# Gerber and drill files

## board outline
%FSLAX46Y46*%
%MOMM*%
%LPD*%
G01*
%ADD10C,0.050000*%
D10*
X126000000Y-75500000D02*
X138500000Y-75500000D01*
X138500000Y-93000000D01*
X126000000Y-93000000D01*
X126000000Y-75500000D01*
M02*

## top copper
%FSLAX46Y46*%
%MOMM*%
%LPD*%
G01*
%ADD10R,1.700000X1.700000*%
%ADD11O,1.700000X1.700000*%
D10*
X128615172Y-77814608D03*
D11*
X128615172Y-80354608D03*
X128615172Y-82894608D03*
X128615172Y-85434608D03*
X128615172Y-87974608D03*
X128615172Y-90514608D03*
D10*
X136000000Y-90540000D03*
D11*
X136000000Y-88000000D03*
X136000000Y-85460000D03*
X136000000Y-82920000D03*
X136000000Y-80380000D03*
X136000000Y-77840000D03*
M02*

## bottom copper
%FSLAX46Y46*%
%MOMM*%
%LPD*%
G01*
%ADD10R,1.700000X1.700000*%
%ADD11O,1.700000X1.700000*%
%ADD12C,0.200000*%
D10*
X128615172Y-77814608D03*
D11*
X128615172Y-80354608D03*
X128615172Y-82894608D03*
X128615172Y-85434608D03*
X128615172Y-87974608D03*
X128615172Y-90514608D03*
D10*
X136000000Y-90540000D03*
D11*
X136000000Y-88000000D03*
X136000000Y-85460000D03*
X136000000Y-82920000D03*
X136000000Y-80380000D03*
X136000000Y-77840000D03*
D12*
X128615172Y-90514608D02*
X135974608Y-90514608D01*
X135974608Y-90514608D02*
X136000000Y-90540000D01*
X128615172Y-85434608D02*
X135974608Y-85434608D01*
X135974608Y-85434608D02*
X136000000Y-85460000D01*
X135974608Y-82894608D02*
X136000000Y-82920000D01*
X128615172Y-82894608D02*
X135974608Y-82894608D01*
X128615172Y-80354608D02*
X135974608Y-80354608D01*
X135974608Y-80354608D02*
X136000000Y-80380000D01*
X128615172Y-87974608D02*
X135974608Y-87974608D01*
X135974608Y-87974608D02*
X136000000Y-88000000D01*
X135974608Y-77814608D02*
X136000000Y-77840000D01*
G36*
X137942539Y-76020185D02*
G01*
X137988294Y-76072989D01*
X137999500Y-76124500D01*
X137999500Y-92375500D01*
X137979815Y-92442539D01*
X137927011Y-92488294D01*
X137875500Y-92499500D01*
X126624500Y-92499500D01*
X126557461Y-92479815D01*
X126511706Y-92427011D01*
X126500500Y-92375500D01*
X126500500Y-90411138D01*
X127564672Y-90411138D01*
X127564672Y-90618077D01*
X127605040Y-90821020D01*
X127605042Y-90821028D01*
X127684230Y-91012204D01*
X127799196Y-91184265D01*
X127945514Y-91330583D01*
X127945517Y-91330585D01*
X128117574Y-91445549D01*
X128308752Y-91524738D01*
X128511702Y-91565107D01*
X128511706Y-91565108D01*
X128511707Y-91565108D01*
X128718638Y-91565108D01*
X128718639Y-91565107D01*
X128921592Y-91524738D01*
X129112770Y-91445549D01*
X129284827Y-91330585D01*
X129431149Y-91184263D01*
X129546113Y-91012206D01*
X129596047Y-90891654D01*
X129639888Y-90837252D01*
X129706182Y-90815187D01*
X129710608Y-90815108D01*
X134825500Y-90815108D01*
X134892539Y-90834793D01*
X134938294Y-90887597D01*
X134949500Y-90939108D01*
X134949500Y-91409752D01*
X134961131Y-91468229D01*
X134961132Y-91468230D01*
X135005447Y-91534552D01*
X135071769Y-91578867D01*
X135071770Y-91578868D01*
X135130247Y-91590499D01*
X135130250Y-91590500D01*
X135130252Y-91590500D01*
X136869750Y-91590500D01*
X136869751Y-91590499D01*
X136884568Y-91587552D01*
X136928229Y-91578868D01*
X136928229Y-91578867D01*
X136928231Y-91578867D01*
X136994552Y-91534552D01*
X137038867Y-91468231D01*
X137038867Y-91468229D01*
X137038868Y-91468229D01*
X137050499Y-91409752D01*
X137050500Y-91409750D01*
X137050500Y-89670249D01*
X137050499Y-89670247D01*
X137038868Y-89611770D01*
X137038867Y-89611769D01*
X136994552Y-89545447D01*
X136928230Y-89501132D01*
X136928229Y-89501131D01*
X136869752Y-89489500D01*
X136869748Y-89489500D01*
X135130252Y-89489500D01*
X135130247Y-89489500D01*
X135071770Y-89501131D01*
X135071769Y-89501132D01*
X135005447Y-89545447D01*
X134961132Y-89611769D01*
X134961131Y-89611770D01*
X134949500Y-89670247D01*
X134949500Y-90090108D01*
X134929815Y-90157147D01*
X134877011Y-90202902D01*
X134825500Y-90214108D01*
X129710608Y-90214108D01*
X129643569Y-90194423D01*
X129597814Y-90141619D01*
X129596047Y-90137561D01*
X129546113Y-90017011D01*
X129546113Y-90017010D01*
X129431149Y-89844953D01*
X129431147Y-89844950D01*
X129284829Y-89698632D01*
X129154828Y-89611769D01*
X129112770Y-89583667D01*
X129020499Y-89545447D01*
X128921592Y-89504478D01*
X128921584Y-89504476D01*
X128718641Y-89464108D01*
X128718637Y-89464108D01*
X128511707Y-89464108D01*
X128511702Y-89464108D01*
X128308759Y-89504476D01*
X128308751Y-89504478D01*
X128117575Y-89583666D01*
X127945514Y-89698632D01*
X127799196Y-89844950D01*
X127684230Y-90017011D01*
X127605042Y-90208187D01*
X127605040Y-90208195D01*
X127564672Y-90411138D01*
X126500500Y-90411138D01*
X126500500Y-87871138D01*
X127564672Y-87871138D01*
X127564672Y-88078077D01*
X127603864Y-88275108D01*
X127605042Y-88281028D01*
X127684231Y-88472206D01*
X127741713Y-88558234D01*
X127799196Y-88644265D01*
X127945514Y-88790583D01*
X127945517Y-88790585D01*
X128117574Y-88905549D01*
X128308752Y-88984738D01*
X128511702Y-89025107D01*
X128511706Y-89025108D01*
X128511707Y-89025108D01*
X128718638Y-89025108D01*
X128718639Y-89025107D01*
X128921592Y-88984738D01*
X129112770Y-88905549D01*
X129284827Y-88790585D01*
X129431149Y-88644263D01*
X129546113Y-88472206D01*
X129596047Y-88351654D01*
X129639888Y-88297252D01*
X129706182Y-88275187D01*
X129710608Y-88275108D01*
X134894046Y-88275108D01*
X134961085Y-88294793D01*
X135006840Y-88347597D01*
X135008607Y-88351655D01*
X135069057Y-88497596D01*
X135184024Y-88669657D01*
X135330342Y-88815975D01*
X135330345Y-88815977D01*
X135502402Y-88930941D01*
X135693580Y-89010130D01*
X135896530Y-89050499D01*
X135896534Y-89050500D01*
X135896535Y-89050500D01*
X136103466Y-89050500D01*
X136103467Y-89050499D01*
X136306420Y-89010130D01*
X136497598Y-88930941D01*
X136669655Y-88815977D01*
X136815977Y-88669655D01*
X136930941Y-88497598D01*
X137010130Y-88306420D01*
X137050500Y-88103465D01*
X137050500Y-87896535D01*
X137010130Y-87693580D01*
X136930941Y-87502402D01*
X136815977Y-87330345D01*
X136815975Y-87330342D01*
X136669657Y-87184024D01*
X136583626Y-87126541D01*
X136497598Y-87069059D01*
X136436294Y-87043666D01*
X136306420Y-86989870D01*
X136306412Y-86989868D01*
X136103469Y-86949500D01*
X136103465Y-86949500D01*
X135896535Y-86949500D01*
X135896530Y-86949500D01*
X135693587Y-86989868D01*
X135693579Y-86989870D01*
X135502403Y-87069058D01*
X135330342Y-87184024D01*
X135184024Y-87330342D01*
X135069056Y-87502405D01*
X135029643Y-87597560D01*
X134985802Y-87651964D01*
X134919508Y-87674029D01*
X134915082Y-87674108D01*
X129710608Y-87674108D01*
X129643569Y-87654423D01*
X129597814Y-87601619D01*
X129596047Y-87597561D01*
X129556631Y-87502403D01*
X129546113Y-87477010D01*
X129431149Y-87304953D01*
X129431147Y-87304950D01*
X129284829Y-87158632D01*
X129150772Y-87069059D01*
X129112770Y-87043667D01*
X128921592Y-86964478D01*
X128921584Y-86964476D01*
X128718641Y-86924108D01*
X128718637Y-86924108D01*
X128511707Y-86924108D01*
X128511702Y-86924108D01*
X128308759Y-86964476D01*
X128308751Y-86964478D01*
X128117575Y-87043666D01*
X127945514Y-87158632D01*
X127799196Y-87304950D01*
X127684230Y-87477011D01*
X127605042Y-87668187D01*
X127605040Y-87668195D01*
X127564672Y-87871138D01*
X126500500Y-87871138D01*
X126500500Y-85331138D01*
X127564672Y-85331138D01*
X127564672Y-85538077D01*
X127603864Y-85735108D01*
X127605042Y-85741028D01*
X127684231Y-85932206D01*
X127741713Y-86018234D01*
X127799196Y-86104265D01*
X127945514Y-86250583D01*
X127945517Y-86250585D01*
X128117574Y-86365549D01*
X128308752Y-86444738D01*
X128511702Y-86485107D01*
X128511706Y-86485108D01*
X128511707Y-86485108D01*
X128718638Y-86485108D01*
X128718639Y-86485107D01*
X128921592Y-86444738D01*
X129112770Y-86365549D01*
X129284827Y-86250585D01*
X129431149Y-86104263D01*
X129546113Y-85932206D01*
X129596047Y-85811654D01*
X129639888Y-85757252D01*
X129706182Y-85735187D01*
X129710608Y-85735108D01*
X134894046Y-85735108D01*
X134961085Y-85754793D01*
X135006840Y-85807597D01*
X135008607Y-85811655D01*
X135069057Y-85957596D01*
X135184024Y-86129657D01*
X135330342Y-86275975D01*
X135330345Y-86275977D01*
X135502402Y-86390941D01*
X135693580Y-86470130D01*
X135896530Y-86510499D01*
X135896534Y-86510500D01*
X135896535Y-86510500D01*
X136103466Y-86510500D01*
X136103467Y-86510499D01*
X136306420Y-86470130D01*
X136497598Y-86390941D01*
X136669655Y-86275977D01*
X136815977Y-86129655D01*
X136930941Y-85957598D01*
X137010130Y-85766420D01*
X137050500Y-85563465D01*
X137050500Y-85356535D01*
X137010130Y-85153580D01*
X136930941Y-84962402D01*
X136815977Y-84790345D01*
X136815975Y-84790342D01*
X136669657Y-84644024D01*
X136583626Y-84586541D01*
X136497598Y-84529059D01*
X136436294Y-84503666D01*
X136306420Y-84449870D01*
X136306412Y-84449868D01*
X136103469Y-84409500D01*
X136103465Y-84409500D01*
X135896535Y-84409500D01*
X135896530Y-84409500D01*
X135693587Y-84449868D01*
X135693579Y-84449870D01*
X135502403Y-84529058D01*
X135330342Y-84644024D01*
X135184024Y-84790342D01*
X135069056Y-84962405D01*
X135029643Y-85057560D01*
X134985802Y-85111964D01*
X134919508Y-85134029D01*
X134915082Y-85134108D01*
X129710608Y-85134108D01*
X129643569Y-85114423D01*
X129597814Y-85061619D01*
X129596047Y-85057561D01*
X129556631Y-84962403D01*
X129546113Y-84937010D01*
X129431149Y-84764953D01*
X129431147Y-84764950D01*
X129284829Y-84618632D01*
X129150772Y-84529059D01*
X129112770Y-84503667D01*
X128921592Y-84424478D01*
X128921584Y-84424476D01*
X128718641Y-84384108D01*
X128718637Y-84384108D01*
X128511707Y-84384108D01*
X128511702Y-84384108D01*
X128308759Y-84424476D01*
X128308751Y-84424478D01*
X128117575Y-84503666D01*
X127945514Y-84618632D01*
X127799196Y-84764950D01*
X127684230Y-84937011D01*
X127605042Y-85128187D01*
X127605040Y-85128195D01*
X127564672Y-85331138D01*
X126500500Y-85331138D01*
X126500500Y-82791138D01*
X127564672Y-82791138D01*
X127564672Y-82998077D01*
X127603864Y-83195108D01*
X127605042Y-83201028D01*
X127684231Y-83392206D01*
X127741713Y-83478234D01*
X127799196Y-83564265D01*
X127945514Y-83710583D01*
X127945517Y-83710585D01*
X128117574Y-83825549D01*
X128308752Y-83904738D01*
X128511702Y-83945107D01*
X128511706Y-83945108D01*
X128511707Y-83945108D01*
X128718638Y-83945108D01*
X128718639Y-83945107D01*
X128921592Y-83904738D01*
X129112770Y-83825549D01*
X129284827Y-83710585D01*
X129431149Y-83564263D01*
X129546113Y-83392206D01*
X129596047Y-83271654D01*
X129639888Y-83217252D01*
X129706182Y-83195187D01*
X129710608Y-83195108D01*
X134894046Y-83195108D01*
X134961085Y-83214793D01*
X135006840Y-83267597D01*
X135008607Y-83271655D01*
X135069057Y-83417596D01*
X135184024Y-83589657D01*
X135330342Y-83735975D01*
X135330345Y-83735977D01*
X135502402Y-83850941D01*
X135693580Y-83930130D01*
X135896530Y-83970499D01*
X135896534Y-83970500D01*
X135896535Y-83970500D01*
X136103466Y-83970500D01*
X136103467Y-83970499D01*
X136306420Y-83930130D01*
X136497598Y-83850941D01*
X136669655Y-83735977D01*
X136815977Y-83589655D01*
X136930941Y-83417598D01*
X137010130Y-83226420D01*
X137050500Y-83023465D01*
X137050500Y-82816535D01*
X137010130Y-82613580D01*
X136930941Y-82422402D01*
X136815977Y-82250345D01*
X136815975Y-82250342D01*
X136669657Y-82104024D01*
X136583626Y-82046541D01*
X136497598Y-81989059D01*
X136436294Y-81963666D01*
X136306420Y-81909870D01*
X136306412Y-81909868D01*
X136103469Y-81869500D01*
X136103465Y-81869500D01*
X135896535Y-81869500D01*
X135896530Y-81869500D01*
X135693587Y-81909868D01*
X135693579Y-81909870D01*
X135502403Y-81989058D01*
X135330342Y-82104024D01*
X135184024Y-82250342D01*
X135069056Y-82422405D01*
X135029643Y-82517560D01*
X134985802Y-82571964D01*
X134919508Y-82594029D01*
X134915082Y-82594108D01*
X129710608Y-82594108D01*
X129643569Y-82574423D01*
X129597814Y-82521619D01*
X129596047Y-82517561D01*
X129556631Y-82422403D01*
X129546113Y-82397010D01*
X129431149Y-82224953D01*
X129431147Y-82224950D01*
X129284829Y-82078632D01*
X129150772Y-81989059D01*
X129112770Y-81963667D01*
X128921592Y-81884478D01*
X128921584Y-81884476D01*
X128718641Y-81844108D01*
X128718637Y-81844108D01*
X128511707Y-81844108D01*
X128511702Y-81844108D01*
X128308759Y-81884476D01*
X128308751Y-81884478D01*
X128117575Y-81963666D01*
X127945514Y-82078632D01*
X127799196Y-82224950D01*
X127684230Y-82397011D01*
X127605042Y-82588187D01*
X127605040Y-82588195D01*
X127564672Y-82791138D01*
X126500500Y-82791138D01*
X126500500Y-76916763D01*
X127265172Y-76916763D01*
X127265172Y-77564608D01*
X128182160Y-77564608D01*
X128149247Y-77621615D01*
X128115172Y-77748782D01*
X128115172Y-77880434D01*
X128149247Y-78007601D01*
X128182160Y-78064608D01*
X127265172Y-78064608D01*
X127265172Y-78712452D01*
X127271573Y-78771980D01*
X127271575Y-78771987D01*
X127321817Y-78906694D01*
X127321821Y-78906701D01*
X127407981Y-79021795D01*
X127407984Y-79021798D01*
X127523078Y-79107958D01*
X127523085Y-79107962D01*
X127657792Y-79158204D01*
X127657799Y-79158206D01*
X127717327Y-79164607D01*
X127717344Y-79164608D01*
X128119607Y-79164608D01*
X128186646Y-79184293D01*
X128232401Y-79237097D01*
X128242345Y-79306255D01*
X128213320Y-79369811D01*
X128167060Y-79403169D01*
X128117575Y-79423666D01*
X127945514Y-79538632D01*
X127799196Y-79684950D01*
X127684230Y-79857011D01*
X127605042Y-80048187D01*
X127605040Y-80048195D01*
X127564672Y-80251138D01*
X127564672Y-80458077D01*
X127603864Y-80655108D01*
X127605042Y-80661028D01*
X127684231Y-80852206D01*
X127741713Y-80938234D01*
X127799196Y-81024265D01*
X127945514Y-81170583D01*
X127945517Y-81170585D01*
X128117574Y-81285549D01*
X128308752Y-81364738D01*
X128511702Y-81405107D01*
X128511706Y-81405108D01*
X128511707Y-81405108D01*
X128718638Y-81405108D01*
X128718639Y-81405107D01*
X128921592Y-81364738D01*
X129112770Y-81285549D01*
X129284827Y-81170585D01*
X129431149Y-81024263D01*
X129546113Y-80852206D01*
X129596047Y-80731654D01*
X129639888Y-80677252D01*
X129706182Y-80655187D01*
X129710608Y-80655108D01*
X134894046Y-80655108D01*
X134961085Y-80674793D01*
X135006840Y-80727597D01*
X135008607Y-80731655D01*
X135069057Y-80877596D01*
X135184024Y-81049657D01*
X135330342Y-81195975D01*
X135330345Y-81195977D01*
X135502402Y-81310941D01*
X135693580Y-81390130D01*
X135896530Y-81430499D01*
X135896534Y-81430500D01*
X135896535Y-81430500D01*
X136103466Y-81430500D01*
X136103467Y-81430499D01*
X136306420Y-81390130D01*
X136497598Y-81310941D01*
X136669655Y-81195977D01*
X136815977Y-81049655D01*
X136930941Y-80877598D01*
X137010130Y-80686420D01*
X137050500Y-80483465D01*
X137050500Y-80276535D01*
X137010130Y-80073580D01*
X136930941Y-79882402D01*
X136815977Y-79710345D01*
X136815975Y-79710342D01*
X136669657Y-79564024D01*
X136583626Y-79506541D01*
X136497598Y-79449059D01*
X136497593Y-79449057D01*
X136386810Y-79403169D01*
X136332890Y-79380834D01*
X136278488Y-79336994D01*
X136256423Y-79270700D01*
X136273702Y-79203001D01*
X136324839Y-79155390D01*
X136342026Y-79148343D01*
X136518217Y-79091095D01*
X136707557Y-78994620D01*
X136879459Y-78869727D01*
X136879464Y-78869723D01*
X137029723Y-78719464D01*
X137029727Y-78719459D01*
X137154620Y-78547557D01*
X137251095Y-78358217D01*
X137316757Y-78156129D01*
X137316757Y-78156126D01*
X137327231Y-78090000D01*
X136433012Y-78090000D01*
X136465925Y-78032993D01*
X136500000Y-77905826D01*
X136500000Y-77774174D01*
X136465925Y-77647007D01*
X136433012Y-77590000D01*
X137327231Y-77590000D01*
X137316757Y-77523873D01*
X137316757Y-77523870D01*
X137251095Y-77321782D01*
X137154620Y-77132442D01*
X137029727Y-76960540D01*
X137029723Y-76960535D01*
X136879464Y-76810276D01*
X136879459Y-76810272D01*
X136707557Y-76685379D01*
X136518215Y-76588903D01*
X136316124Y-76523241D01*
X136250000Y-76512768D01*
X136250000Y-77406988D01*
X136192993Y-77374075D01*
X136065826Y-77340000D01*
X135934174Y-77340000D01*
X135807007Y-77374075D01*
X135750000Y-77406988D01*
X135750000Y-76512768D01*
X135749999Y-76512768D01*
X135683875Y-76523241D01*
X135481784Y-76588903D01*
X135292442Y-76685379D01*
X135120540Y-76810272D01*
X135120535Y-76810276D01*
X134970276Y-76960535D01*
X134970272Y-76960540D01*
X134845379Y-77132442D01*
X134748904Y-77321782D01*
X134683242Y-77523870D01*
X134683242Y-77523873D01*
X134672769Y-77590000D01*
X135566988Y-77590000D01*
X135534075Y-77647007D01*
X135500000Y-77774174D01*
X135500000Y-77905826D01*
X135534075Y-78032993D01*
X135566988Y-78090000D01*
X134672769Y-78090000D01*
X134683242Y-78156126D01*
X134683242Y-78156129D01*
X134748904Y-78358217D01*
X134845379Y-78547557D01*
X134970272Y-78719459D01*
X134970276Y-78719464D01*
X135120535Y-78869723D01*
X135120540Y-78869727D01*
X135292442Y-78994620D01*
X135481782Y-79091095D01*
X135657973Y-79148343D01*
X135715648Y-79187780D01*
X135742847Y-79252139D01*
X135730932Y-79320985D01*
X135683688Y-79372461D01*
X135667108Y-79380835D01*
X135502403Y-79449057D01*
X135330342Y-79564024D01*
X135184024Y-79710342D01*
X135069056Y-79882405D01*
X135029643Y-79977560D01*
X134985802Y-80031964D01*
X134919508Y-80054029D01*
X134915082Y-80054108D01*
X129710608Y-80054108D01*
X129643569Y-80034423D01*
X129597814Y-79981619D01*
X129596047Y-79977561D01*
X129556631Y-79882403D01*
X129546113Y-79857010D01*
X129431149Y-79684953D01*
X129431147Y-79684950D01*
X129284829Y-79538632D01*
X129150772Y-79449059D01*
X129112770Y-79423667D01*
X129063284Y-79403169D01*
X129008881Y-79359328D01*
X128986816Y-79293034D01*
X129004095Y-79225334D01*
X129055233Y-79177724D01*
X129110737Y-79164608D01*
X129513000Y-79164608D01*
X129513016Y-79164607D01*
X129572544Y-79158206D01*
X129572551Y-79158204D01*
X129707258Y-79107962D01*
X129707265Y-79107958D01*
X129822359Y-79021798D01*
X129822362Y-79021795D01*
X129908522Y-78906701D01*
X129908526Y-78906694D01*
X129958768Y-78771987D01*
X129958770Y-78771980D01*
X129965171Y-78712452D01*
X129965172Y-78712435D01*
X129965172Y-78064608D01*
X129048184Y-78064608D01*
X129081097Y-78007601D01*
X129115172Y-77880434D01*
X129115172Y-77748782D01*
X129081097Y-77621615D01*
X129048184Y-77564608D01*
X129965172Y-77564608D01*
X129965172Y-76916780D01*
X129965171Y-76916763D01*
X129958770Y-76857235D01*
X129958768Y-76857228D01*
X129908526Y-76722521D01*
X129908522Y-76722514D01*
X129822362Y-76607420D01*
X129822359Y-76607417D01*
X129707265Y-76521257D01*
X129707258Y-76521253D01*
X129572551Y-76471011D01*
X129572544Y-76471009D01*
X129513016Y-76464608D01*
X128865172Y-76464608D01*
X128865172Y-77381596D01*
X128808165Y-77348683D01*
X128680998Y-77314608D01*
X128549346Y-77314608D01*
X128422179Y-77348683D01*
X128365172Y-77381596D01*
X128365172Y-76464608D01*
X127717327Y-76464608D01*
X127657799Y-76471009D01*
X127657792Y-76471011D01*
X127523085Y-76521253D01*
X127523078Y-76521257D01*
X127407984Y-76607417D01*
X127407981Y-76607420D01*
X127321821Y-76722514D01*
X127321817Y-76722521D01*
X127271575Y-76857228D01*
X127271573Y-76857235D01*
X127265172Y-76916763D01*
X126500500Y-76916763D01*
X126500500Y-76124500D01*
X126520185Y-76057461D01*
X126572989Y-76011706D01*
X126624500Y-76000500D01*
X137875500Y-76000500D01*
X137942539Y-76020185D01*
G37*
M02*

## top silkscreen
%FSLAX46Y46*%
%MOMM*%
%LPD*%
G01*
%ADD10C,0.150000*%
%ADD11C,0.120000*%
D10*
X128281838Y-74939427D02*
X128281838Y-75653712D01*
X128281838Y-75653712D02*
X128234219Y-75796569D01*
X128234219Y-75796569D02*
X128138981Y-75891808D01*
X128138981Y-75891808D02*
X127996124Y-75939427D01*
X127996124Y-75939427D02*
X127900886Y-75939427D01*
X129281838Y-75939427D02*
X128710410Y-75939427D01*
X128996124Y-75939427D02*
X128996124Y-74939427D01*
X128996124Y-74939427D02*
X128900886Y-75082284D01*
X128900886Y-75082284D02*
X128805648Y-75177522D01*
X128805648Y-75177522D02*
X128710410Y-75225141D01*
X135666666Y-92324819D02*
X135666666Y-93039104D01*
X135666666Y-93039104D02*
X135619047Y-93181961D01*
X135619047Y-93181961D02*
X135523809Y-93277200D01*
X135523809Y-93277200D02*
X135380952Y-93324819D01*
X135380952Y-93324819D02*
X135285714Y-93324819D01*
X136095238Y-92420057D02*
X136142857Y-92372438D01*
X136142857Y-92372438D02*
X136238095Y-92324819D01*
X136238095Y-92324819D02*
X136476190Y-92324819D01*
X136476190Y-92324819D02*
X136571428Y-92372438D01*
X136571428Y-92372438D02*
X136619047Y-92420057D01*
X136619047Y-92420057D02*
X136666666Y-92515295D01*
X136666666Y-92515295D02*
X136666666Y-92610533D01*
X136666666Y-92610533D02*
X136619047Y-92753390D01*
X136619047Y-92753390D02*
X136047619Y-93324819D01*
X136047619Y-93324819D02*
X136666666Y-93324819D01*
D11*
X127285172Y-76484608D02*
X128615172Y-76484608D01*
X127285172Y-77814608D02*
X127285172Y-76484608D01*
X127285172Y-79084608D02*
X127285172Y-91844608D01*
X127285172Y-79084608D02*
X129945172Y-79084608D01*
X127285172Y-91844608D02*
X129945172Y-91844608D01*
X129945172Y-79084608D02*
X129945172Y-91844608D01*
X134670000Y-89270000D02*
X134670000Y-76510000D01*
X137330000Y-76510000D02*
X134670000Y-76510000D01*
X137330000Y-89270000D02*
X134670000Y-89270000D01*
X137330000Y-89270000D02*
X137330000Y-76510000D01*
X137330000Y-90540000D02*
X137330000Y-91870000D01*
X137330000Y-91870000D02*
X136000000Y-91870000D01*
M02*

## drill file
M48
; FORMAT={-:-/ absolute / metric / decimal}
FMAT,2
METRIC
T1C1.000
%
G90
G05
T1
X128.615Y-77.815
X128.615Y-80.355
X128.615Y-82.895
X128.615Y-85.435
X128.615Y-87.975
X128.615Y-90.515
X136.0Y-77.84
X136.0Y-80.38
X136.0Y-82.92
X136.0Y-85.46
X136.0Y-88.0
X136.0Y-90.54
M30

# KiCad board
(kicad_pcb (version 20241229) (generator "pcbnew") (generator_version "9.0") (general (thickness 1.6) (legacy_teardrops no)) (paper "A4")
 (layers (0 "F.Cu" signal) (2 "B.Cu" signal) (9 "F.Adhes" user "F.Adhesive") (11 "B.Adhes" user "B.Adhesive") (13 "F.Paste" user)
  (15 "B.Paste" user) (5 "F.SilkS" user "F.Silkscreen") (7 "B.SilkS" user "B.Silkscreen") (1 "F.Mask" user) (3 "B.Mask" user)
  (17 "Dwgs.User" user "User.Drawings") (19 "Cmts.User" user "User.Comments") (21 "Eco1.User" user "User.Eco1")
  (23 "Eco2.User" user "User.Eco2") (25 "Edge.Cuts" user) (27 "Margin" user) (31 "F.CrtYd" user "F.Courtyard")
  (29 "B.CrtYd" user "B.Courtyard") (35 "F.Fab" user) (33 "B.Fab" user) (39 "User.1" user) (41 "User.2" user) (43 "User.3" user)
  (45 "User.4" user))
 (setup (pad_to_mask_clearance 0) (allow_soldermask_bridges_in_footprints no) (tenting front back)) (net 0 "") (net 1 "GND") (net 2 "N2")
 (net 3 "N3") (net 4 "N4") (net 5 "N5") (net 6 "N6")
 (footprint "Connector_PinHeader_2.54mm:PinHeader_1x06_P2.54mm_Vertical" (layer "F.Cu") (at 128.615172 77.814608)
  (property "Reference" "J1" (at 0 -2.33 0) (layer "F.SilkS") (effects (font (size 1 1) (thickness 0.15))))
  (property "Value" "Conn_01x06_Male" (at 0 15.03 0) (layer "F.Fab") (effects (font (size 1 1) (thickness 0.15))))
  (fp_line (start -1.33 -1.33) (end 0 -1.33) (stroke (width 0.12) (type solid)) (layer "F.SilkS"))
  (fp_line (start -1.33 0) (end -1.33 -1.33) (stroke (width 0.12) (type solid)) (layer "F.SilkS"))
  (fp_line (start -1.33 1.27) (end -1.33 14.03) (stroke (width 0.12) (type solid)) (layer "F.SilkS"))
  (fp_line (start -1.33 1.27) (end 1.33 1.27) (stroke (width 0.12) (type solid)) (layer "F.SilkS"))
  (fp_line (start -1.33 14.03) (end 1.33 14.03) (stroke (width 0.12) (type solid)) (layer "F.SilkS"))
  (fp_line (start 1.33 1.27) (end 1.33 14.03) (stroke (width 0.12) (type solid)) (layer "F.SilkS"))
  (pad "1" thru_hole rect (at 0 0) (size 1.7 1.7) (drill 1) (layers "*.Cu" "*.Mask") (remove_unused_layers no) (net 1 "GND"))
  (pad "2" thru_hole oval (at 0 2.54) (size 1.7 1.7) (drill 1) (layers "*.Cu" "*.Mask") (remove_unused_layers no) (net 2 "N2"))
  (pad "3" thru_hole oval (at 0 5.08) (size 1.7 1.7) (drill 1) (layers "*.Cu" "*.Mask") (remove_unused_layers no) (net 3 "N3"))
  (pad "4" thru_hole oval (at 0 7.62) (size 1.7 1.7) (drill 1) (layers "*.Cu" "*.Mask") (remove_unused_layers no) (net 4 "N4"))
  (pad "5" thru_hole oval (at 0 10.16) (size 1.7 1.7) (drill 1) (layers "*.Cu" "*.Mask") (remove_unused_layers no) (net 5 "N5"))
  (pad "6" thru_hole oval (at 0 12.7) (size 1.7 1.7) (drill 1) (layers "*.Cu" "*.Mask") (remove_unused_layers no) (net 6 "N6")))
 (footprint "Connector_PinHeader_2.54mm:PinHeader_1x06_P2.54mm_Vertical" (layer "F.Cu") (at 136 90.54 180)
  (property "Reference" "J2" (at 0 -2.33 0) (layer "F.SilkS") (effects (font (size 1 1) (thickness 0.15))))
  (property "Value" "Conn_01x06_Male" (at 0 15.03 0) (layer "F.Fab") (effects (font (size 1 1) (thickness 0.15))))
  (fp_line (start 1.33 1.27) (end 1.33 14.03) (stroke (width 0.12) (type solid)) (layer "F.SilkS"))
  (fp_line (start -1.33 14.03) (end 1.33 14.03) (stroke (width 0.12) (type solid)) (layer "F.SilkS"))
  (fp_line (start -1.33 1.27) (end 1.33 1.27) (stroke (width 0.12) (type solid)) (layer "F.SilkS"))
  (fp_line (start -1.33 1.27) (end -1.33 14.03) (stroke (width 0.12) (type solid)) (layer "F.SilkS"))
  (fp_line (start -1.33 0) (end -1.33 -1.33) (stroke (width 0.12) (type solid)) (layer "F.SilkS"))
  (fp_line (start -1.33 -1.33) (end 0 -1.33) (stroke (width 0.12) (type solid)) (layer "F.SilkS"))
  (pad "1" thru_hole rect (at 0 0 180) (size 1.7 1.7) (drill 1) (layers "*.Cu" "*.Mask") (remove_unused_layers no) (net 6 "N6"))
  (pad "2" thru_hole oval (at 0 2.54 180) (size 1.7 1.7) (drill 1) (layers "*.Cu" "*.Mask") (remove_unused_layers no) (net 5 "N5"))
  (pad "3" thru_hole oval (at 0 5.08 180) (size 1.7 1.7) (drill 1) (layers "*.Cu" "*.Mask") (remove_unused_layers no) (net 4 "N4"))
  (pad "4" thru_hole oval (at 0 7.62 180) (size 1.7 1.7) (drill 1) (layers "*.Cu" "*.Mask") (remove_unused_layers no) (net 3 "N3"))
  (pad "5" thru_hole oval (at 0 10.16 180) (size 1.7 1.7) (drill 1) (layers "*.Cu" "*.Mask") (remove_unused_layers no) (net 2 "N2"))
  (pad "6" thru_hole oval (at 0 12.7 180) (size 1.7 1.7) (drill 1) (layers "*.Cu" "*.Mask") (remove_unused_layers no) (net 1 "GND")))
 (gr_rect (start 126 75.5) (end 138.5 93) (stroke (width 0.05) (type default)) (fill no) (layer "Edge.Cuts"))
 (segment (start 128.615172 90.514608) (end 135.974608 90.514608) (width 0.2) (layer "B.Cu") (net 6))
 (segment (start 135.974608 90.514608) (end 136 90.54) (width 0.2) (layer "B.Cu") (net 6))
 (segment (start 128.615172 85.434608) (end 135.974608 85.434608) (width 0.2) (layer "B.Cu") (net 4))
 (segment (start 135.974608 85.434608) (end 136 85.46) (width 0.2) (layer "B.Cu") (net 4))
 (segment (start 135.974608 82.894608) (end 136 82.92) (width 0.2) (layer "B.Cu") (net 3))
 (segment (start 128.615172 82.894608) (end 135.974608 82.894608) (width 0.2) (layer "B.Cu") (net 3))
 (segment (start 128.615172 80.354608) (end 135.974608 80.354608) (width 0.2) (layer "B.Cu") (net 2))
 (segment (start 135.974608 80.354608) (end 136 80.38) (width 0.2) (layer "B.Cu") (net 2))
 (segment (start 128.615172 87.974608) (end 135.974608 87.974608) (width 0.2) (layer "B.Cu") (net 5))
 (segment (start 135.974608 87.974608) (end 136 88) (width 0.2) (layer "B.Cu") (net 5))
 (segment (start 135.974608 77.814608) (end 136 77.84) (width 0.2) (layer "B.Cu") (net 1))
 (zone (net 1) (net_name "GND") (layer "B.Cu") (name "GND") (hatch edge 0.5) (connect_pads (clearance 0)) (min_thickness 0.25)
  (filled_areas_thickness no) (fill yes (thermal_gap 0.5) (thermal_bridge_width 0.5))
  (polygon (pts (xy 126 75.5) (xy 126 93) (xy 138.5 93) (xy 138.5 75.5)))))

